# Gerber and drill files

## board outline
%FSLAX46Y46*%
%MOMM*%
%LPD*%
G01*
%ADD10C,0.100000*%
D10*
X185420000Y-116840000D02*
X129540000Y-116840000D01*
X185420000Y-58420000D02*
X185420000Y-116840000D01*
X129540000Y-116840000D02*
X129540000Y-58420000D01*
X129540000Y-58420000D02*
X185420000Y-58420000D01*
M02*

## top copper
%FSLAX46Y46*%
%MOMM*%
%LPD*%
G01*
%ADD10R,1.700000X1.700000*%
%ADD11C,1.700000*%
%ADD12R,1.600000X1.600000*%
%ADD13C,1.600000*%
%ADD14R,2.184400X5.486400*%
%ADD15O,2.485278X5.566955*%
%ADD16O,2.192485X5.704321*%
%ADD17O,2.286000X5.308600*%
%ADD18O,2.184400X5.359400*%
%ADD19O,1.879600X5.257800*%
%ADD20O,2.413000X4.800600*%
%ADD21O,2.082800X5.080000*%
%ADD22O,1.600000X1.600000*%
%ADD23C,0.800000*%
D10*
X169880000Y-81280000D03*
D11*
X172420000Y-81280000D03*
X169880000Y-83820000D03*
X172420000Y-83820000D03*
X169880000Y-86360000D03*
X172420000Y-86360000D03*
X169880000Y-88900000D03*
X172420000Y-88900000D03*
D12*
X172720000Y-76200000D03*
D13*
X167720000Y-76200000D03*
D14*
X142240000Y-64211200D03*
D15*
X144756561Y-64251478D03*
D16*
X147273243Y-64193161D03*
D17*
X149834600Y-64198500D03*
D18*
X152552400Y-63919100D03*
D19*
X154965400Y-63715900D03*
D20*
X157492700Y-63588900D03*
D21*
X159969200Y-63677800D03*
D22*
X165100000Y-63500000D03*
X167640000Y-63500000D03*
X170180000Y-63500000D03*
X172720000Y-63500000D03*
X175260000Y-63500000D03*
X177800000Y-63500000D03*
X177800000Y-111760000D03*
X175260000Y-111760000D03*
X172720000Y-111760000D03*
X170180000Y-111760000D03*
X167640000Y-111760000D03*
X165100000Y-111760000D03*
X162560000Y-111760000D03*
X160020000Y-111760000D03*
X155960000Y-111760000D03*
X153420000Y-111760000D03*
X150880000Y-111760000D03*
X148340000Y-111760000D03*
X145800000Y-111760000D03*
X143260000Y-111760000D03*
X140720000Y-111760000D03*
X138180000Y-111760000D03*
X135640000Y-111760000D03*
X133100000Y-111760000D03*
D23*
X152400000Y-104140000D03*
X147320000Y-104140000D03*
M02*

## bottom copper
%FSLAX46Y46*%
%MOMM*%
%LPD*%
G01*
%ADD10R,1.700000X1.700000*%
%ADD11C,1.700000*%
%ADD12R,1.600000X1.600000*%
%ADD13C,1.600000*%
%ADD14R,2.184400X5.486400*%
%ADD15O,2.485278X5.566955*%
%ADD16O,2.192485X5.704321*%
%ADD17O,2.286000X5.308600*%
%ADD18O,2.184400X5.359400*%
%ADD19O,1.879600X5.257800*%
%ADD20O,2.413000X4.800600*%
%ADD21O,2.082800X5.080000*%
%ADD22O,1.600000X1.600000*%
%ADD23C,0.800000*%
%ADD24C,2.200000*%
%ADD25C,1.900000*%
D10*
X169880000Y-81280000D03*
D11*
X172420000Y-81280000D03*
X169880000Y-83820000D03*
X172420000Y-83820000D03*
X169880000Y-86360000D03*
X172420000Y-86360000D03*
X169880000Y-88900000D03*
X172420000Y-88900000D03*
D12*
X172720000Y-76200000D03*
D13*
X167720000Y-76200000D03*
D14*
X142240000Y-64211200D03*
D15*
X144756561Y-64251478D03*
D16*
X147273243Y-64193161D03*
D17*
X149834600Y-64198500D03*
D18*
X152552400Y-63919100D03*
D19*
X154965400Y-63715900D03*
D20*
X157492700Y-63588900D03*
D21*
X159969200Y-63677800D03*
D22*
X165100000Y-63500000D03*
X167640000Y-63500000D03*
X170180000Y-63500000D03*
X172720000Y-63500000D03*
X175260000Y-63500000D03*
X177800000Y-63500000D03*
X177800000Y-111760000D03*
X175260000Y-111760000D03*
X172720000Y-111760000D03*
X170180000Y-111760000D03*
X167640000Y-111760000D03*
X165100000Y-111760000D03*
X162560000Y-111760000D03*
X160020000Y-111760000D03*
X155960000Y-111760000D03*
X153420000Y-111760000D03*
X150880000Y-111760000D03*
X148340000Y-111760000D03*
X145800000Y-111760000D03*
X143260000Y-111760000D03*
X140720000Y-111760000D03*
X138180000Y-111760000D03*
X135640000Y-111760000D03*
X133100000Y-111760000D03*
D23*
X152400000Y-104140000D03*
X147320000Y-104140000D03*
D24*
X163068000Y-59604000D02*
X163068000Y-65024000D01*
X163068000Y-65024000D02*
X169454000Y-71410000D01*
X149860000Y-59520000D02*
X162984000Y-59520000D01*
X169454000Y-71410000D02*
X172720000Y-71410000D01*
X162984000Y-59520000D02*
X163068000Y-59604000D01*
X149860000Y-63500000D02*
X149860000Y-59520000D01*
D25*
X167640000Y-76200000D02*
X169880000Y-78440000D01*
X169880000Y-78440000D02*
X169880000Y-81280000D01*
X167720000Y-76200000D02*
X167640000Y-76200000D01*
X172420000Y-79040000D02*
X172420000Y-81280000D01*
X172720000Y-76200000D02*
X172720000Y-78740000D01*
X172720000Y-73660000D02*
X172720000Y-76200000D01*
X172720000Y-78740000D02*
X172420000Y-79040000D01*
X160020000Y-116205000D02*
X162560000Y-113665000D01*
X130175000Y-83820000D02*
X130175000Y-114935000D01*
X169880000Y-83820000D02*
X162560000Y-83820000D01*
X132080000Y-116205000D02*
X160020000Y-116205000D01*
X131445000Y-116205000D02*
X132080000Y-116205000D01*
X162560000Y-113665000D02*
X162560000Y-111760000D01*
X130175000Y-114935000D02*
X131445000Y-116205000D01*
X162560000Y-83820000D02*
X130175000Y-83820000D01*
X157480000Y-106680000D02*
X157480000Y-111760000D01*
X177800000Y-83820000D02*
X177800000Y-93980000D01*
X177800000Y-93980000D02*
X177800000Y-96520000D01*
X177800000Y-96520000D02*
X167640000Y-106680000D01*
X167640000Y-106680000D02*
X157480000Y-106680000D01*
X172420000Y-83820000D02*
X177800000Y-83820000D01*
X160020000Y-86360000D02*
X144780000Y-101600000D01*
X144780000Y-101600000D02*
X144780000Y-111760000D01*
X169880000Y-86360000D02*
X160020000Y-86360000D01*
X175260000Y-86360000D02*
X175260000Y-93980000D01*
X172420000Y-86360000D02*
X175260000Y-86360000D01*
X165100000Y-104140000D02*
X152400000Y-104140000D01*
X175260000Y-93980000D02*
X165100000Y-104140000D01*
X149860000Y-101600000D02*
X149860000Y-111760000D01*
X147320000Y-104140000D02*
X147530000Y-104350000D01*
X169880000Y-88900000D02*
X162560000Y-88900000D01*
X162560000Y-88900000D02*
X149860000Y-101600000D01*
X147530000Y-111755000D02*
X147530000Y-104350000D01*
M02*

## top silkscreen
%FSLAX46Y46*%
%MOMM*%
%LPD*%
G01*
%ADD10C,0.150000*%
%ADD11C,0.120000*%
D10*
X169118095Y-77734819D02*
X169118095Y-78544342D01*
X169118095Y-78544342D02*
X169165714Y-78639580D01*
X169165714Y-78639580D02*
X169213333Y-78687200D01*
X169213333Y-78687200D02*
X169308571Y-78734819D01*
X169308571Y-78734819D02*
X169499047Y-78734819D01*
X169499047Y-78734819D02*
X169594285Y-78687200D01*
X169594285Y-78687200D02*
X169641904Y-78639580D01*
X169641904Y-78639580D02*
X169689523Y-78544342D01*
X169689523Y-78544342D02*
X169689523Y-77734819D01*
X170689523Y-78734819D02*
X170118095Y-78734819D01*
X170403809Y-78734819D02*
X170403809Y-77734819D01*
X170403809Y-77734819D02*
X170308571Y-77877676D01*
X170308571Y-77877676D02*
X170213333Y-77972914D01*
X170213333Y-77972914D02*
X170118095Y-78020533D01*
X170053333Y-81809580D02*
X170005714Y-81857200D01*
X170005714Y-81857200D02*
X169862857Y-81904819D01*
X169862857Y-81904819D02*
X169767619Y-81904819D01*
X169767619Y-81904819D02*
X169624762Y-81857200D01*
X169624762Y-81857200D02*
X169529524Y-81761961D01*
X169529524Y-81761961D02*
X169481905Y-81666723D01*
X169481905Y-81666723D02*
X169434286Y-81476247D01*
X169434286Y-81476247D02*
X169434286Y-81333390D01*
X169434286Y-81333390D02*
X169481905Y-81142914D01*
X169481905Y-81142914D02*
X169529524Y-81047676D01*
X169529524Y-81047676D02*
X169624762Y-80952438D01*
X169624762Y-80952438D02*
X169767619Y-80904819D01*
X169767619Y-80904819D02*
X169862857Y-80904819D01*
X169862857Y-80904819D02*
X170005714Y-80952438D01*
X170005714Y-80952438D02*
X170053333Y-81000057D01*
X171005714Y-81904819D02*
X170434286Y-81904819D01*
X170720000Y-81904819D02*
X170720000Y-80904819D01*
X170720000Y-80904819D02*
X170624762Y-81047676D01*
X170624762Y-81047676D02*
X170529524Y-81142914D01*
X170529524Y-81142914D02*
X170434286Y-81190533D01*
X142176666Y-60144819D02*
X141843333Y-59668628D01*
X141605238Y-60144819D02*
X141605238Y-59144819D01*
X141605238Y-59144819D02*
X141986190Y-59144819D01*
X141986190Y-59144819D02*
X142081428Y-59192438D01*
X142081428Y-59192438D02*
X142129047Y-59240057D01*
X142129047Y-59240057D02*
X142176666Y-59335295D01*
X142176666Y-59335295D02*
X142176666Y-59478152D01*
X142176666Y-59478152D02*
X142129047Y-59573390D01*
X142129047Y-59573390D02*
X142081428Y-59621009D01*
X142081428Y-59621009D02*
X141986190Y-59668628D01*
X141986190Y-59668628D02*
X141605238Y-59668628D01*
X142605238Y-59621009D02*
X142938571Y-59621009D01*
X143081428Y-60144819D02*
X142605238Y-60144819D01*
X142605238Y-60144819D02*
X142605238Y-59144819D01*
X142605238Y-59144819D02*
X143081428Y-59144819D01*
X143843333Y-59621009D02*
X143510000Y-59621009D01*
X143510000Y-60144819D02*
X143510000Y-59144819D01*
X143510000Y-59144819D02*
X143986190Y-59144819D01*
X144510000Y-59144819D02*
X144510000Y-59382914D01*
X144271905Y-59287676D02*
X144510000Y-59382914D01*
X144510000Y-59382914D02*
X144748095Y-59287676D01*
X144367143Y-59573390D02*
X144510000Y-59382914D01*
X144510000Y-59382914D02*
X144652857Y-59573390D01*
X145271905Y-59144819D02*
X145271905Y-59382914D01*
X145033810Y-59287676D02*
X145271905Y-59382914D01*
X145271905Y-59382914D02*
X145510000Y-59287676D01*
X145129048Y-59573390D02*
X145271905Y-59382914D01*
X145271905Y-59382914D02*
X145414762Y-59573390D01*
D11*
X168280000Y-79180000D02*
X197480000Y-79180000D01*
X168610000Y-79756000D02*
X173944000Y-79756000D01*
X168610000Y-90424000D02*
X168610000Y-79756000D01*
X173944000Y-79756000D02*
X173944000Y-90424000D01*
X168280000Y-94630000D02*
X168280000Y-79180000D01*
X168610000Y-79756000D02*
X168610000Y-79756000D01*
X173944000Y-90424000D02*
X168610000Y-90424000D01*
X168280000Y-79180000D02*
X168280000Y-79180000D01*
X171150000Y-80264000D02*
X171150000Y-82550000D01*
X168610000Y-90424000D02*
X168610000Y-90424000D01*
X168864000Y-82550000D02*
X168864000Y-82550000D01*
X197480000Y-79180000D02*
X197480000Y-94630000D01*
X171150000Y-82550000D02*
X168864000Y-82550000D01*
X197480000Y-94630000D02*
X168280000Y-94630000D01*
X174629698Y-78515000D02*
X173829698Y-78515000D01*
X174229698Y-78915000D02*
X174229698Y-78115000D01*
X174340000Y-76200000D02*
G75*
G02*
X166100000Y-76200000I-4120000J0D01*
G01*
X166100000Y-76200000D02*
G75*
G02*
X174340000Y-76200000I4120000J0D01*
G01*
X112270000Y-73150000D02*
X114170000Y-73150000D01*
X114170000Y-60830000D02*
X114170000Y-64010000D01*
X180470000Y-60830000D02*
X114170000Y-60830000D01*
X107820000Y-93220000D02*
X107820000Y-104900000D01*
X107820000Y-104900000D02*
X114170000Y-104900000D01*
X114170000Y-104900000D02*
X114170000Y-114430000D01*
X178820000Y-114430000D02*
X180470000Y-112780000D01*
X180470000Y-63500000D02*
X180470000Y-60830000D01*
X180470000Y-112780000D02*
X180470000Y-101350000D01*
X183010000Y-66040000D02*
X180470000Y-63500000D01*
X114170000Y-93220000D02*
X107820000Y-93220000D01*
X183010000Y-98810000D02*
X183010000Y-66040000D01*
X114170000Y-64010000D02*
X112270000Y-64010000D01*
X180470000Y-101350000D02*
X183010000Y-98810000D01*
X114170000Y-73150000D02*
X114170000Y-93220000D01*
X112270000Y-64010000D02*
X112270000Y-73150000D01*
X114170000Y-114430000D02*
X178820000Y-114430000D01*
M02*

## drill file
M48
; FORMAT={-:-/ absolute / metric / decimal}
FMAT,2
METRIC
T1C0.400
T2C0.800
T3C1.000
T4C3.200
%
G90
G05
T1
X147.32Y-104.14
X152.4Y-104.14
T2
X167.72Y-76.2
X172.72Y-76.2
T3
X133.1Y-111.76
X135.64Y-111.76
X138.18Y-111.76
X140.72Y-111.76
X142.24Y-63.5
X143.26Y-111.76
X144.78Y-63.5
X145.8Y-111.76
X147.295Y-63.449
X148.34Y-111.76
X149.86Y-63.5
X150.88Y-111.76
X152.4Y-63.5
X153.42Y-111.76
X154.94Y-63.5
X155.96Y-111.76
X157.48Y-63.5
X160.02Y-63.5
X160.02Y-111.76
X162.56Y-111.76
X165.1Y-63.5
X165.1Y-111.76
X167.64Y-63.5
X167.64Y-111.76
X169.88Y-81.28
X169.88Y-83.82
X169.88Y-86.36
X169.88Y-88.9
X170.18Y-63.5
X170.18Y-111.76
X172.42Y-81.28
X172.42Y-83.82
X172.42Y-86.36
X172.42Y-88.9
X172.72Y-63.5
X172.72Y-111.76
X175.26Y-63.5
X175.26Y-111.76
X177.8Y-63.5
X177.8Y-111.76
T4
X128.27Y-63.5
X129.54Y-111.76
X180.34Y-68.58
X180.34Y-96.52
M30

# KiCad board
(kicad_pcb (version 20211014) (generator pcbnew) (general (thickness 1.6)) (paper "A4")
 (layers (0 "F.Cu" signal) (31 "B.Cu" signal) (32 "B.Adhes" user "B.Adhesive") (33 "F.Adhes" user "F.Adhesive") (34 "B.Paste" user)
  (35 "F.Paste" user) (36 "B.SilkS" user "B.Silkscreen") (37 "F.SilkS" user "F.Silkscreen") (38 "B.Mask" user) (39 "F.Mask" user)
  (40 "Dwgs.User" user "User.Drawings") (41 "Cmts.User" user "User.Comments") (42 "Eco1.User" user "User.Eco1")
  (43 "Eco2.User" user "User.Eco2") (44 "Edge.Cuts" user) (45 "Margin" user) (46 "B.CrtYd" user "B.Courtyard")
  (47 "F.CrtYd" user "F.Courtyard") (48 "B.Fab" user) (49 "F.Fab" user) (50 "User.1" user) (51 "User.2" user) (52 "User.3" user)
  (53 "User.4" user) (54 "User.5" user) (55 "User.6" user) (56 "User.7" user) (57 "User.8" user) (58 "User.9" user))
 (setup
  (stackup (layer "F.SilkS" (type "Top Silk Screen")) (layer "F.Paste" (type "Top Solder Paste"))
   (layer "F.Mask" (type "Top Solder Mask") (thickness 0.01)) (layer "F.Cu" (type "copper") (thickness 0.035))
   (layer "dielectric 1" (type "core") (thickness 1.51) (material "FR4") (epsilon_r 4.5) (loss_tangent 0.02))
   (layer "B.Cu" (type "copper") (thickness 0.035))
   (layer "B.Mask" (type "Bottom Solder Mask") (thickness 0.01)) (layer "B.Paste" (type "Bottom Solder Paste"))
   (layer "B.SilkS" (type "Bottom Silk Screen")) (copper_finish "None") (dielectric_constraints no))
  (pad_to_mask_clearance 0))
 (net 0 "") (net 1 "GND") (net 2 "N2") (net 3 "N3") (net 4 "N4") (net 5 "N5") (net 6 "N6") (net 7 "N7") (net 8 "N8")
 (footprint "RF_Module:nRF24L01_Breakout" (layer "F.Cu") (at 169.88 81.28)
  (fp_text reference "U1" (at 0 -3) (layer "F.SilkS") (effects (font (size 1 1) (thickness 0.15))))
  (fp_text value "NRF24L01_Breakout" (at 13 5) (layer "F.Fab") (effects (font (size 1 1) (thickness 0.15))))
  (fp_line (start -1.6 -2.1) (end 27.6 -2.1) (layer "F.SilkS") (width 0.12))
  (fp_line (start -1.27 -1.524) (end 4.064 -1.524) (layer "F.SilkS") (width 0.12))
  (fp_line (start -1.27 9.144) (end -1.27 -1.524) (layer "F.SilkS") (width 0.12))
  (fp_line (start 4.064 -1.524) (end 4.064 9.144) (layer "F.SilkS") (width 0.12))
  (fp_line (start -1.6 13.35) (end -1.6 -2.1) (layer "F.SilkS") (width 0.12))
  (fp_line (start -1.27 -1.524) (end -1.27 -1.524) (layer "F.SilkS") (width 0.12))
  (fp_line (start 4.064 9.144) (end -1.27 9.144) (layer "F.SilkS") (width 0.12))
  (fp_line (start -1.6 -2.1) (end -1.6 -2.1) (layer "F.SilkS") (width 0.12))
  (fp_line (start 1.27 -1.016) (end 1.27 1.27) (layer "F.SilkS") (width 0.12))
  (fp_line (start -1.27 9.144) (end -1.27 9.144) (layer "F.SilkS") (width 0.12))
  (fp_line (start -1.016 1.27) (end -1.016 1.27) (layer "F.SilkS") (width 0.12))
  (fp_line (start 27.6 -2.1) (end 27.6 13.35) (layer "F.SilkS") (width 0.12))
  (fp_line (start 1.27 1.27) (end -1.016 1.27) (layer "F.SilkS") (width 0.12))
  (fp_line (start 27.6 13.35) (end -1.6 13.35) (layer "F.SilkS") (width 0.12))
  (pad "1" thru_hole rect (at 0 0) (size 1.7 1.7) (drill 1) (layers *.Cu *.Mask) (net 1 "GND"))
  (pad "2" thru_hole circle (at 2.54 0) (size 1.7 1.7) (drill 1) (layers *.Cu *.Mask) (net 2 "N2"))
  (pad "3" thru_hole circle (at 0 2.54) (size 1.7 1.7) (drill 1) (layers *.Cu *.Mask) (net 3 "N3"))
  (pad "4" thru_hole circle (at 2.54 2.54) (size 1.7 1.7) (drill 1) (layers *.Cu *.Mask) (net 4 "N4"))
  (pad "5" thru_hole circle (at 0 5.08) (size 1.7 1.7) (drill 1) (layers *.Cu *.Mask) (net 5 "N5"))
  (pad "6" thru_hole circle (at 2.54 5.08) (size 1.7 1.7) (drill 1) (layers *.Cu *.Mask) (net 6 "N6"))
  (pad "7" thru_hole circle (at 0 7.62) (size 1.7 1.7) (drill 1) (layers *.Cu *.Mask) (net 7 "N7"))
  (pad "8" thru_hole circle (at 2.54 7.62) (size 1.7 1.7) (drill 1) (layers *.Cu *.Mask) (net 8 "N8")))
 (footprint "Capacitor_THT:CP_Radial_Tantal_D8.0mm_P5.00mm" (layer "F.Cu") (at 172.72 76.2 180)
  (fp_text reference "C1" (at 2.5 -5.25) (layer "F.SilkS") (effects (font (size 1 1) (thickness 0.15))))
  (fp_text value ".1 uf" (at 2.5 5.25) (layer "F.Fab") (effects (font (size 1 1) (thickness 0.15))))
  (fp_line (start -1.909698 -2.315) (end -1.109698 -2.315) (layer "F.SilkS") (width 0.12))
  (fp_line (start -1.509698 -2.715) (end -1.509698 -1.915) (layer "F.SilkS") (width 0.12))
  (fp_circle (center 2.5 0) (end 6.62 0) (layer "F.SilkS") (width 0.12) (fill none))
  (pad "1" thru_hole rect (at 0 0 180) (size 1.6 1.6) (drill 0.8) (layers *.Cu *.Mask) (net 2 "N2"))
  (pad "2" thru_hole circle (at 5 0 180) (size 1.6 1.6) (drill 0.8) (layers *.Cu *.Mask) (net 1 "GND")))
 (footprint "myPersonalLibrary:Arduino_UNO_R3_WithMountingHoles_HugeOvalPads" (layer "F.Cu") (at 142.24 63.5)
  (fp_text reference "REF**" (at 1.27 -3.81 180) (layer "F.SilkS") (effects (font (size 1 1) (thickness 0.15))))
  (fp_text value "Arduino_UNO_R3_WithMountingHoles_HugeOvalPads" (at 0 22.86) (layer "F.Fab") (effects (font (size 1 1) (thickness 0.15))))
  (fp_line (start -29.97 9.65) (end -28.07 9.65) (layer "F.SilkS") (width 0.12))
  (fp_line (start -28.07 -2.67) (end -28.07 0.51) (layer "F.SilkS") (width 0.12))
  (fp_line (start 38.23 -2.67) (end -28.07 -2.67) (layer "F.SilkS") (width 0.12))
  (fp_line (start -34.42 29.72) (end -34.42 41.4) (layer "F.SilkS") (width 0.12))
  (fp_line (start -34.42 41.4) (end -28.07 41.4) (layer "F.SilkS") (width 0.12))
  (fp_line (start -28.07 41.4) (end -28.07 50.93) (layer "F.SilkS") (width 0.12))
  (fp_line (start 36.58 50.93) (end 38.23 49.28) (layer "F.SilkS") (width 0.12))
  (fp_line (start 38.23 0) (end 38.23 -2.67) (layer "F.SilkS") (width 0.12))
  (fp_line (start 38.23 49.28) (end 38.23 37.85) (layer "F.SilkS") (width 0.12))
  (fp_line (start 40.77 2.54) (end 38.23 0) (layer "F.SilkS") (width 0.12))
  (fp_line (start -28.07 29.72) (end -34.42 29.72) (layer "F.SilkS") (width 0.12))
  (fp_line (start 40.77 35.31) (end 40.77 2.54) (layer "F.SilkS") (width 0.12))
  (fp_line (start -28.07 0.51) (end -29.97 0.51) (layer "F.SilkS") (width 0.12))
  (fp_line (start 38.23 37.85) (end 40.77 35.31) (layer "F.SilkS") (width 0.12))
  (fp_line (start -28.07 9.65) (end -28.07 29.72) (layer "F.SilkS") (width 0.12))
  (fp_line (start -29.97 0.51) (end -29.97 9.65) (layer "F.SilkS") (width 0.12))
  (fp_line (start -28.07 50.93) (end 36.58 50.93) (layer "F.SilkS") (width 0.12))
  (pad "" np_thru_hole circle (at -12.7 48.26 90) (size 3.2 3.2) (drill 3.2) (layers *.Cu *.Mask))
  (pad "" np_thru_hole circle (at 38.1 5.08 90) (size 3.2 3.2) (drill 3.2) (layers *.Cu *.Mask))
  (pad "" np_thru_hole circle (at -13.97 0 90) (size 3.2 3.2) (drill 3.2) (layers *.Cu *.Mask))
  (pad "" np_thru_hole circle (at 38.1 33.02 90) (size 3.2 3.2) (drill 3.2) (layers *.Cu *.Mask))
  (pad "1" thru_hole rect (at 0 0 90) (size 5.4864 2.1844) (drill 1 (offset -0.7112 0)) (layers *.Cu *.Mask))
  (pad "2" thru_hole oval (at 2.54 0 90) (size 5.566955 2.485278) (drill 1 (offset -0.751478 -0.023439)) (layers *.Cu *.Mask))
  (pad "3" thru_hole oval (at 5.0546 -0.0508 90) (size 5.704321 2.192485) (drill 1 (offset -0.743961 -0.021357)) (layers *.Cu *.Mask))
  (pad "4" thru_hole oval (at 7.62 0 90) (size 5.3086 2.286) (drill 1 (offset -0.6985 -0.0254)) (layers *.Cu *.Mask))
  (pad "5" thru_hole oval (at 10.16 0 90) (size 5.3594 2.1844) (drill 1 (offset -0.4191 0.1524)) (layers *.Cu *.Mask))
  (pad "6" thru_hole oval (at 12.7 0 90) (size 5.2578 1.8796) (drill 1 (offset -0.2159 0.0254)) (layers *.Cu *.Mask))
  (pad "7" thru_hole oval (at 15.24 0 90) (size 4.8006 2.413) (drill 1 (offset -0.0889 0.0127)) (layers *.Cu *.Mask))
  (pad "8" thru_hole oval (at 17.78 0 90) (size 5.08 2.0828) (drill 1 (offset -0.1778 -0.0508)) (layers *.Cu *.Mask))
  (pad "9" thru_hole oval (at 22.86 0 90) (size 1.6 1.6) (drill 1) (layers *.Cu *.Mask))
  (pad "10" thru_hole oval (at 25.4 0 90) (size 1.6 1.6) (drill 1) (layers *.Cu *.Mask))
  (pad "11" thru_hole oval (at 27.94 0 90) (size 1.6 1.6) (drill 1) (layers *.Cu *.Mask))
  (pad "12" thru_hole oval (at 30.48 0 90) (size 1.6 1.6) (drill 1) (layers *.Cu *.Mask))
  (pad "13" thru_hole oval (at 33.02 0 90) (size 1.6 1.6) (drill 1) (layers *.Cu *.Mask))
  (pad "14" thru_hole oval (at 35.56 0 90) (size 1.6 1.6) (drill 1) (layers *.Cu *.Mask))
  (pad "15" thru_hole oval (at 35.56 48.26 90) (size 1.6 1.6) (drill 1) (layers *.Cu *.Mask))
  (pad "16" thru_hole oval (at 33.02 48.26 90) (size 1.6 1.6) (drill 1) (layers *.Cu *.Mask))
  (pad "17" thru_hole oval (at 30.48 48.26 90) (size 1.6 1.6) (drill 1) (layers *.Cu *.Mask))
  (pad "18" thru_hole oval (at 27.94 48.26 90) (size 1.6 1.6) (drill 1) (layers *.Cu *.Mask))
  (pad "19" thru_hole oval (at 25.4 48.26 90) (size 1.6 1.6) (drill 1) (layers *.Cu *.Mask))
  (pad "20" thru_hole oval (at 22.86 48.26 90) (size 1.6 1.6) (drill 1) (layers *.Cu *.Mask))
  (pad "21" thru_hole oval (at 20.32 48.26 90) (size 1.6 1.6) (drill 1) (layers *.Cu *.Mask))
  (pad "22" thru_hole oval (at 17.78 48.26 90) (size 1.6 1.6) (drill 1) (layers *.Cu *.Mask))
  (pad "23" thru_hole oval (at 13.72 48.26 90) (size 1.6 1.6) (drill 1) (layers *.Cu *.Mask))
  (pad "24" thru_hole oval (at 11.18 48.26 90) (size 1.6 1.6) (drill 1) (layers *.Cu *.Mask))
  (pad "25" thru_hole oval (at 8.64 48.26 90) (size 1.6 1.6) (drill 1) (layers *.Cu *.Mask))
  (pad "26" thru_hole oval (at 6.1 48.26 90) (size 1.6 1.6) (drill 1) (layers *.Cu *.Mask))
  (pad "27" thru_hole oval (at 3.56 48.26 90) (size 1.6 1.6) (drill 1) (layers *.Cu *.Mask))
  (pad "28" thru_hole oval (at 1.02 48.26 90) (size 1.6 1.6) (drill 1) (layers *.Cu *.Mask))
  (pad "29" thru_hole oval (at -1.52 48.26 90) (size 1.6 1.6) (drill 1) (layers *.Cu *.Mask))
  (pad "30" thru_hole oval (at -4.06 48.26 90) (size 1.6 1.6) (drill 1) (layers *.Cu *.Mask))
  (pad "31" thru_hole oval (at -6.6 48.26 90) (size 1.6 1.6) (drill 1) (layers *.Cu *.Mask))
  (pad "32" thru_hole oval (at -9.14 48.26 90) (size 1.6 1.6) (drill 1) (layers *.Cu *.Mask)))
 (gr_line (start 185.42 116.84) (end 129.54 116.84) (layer "Edge.Cuts") (width 0.1))
 (gr_line (start 185.42 58.42) (end 185.42 116.84) (layer "Edge.Cuts") (width 0.1))
 (gr_line (start 129.54 116.84) (end 129.54 58.42) (layer "Edge.Cuts") (width 0.1))
 (gr_line (start 129.54 58.42) (end 185.42 58.42) (layer "Edge.Cuts") (width 0.1))
 (segment (start 163.068 59.604) (end 163.068 65.024) (width 2.2) (layer "B.Cu") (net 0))
 (segment (start 163.068 65.024) (end 169.454 71.41) (width 2.2) (layer "B.Cu") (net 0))
 (segment (start 149.86 59.52) (end 162.984 59.52) (width 2.2) (layer "B.Cu") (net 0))
 (segment (start 169.454 71.41) (end 172.72 71.41) (width 2.2) (layer "B.Cu") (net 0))
 (segment (start 162.984 59.52) (end 163.068 59.604) (width 2.2) (layer "B.Cu") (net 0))
 (segment (start 149.86 63.5) (end 149.86 59.52) (width 2.2) (layer "B.Cu") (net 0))
 (segment (start 167.64 76.2) (end 169.88 78.44) (width 1.9) (layer "B.Cu") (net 1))
 (segment (start 169.88 78.44) (end 169.88 81.28) (width 1.9) (layer "B.Cu") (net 1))
 (segment (start 167.72 76.2) (end 167.64 76.2) (width 1.9) (layer "B.Cu") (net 1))
 (segment (start 172.42 79.04) (end 172.42 81.28) (width 1.9) (layer "B.Cu") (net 2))
 (segment (start 172.72 76.2) (end 172.72 78.74) (width 1.9) (layer "B.Cu") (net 2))
 (segment (start 172.72 73.66) (end 172.72 76.2) (width 1.9) (layer "B.Cu") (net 2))
 (segment (start 172.72 78.74) (end 172.42 79.04) (width 1.9) (layer "B.Cu") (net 2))
 (segment (start 160.02 116.205) (end 162.56 113.665) (width 1.9) (layer "B.Cu") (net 3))
 (segment (start 130.175 83.82) (end 130.175 114.935) (width 1.9) (layer "B.Cu") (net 3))
 (segment (start 169.88 83.82) (end 162.56 83.82) (width 1.9) (layer "B.Cu") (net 3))
 (segment (start 132.08 116.205) (end 160.02 116.205) (width 1.9) (layer "B.Cu") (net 3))
 (segment (start 131.445 116.205) (end 132.08 116.205) (width 1.9) (layer "B.Cu") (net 3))
 (segment (start 162.56 113.665) (end 162.56 111.76) (width 1.9) (layer "B.Cu") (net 3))
 (segment (start 130.175 114.935) (end 131.445 116.205) (width 1.9) (layer "B.Cu") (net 3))
 (segment (start 162.56 83.82) (end 130.175 83.82) (width 1.9) (layer "B.Cu") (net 3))
 (segment (start 157.48 106.68) (end 157.48 111.76) (width 1.9) (layer "B.Cu") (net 4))
 (segment (start 177.8 83.82) (end 177.8 93.98) (width 1.9) (layer "B.Cu") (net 4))
 (segment (start 177.8 93.98) (end 177.8 96.52) (width 1.9) (layer "B.Cu") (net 4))
 (segment (start 177.8 96.52) (end 167.64 106.68) (width 1.9) (layer "B.Cu") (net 4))
 (segment (start 167.64 106.68) (end 157.48 106.68) (width 1.9) (layer "B.Cu") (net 4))
 (segment (start 172.42 83.82) (end 177.8 83.82) (width 1.9) (layer "B.Cu") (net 4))
 (segment (start 160.02 86.36) (end 144.78 101.6) (width 1.9) (layer "B.Cu") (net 5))
 (segment (start 144.78 101.6) (end 144.78 111.76) (width 1.9) (layer "B.Cu") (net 5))
 (segment (start 169.88 86.36) (end 160.02 86.36) (width 1.9) (layer "B.Cu") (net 5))
 (via (at 152.4 104.14) (size 0.8) (drill 0.4) (layers "F.Cu" "B.Cu") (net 6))
 (segment (start 175.26 86.36) (end 175.26 93.98) (width 1.9) (layer "B.Cu") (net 6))
 (segment (start 172.42 86.36) (end 175.26 86.36) (width 1.9) (layer "B.Cu") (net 6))
 (segment (start 165.1 104.14) (end 152.4 104.14) (width 1.9) (layer "B.Cu") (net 6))
 (segment (start 175.26 93.98) (end 165.1 104.14) (width 1.9) (layer "B.Cu") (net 6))
 (via (at 147.32 104.14) (size 0.8) (drill 0.4) (layers "F.Cu" "B.Cu") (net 7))
 (segment (start 149.86 101.6) (end 149.86 111.76) (width 1.9) (layer "B.Cu") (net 7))
 (segment (start 147.32 104.14) (end 147.53 104.35) (width 1.9) (layer "B.Cu") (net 7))
 (segment (start 169.88 88.9) (end 162.56 88.9) (width 1.9) (layer "B.Cu") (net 7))
 (segment (start 162.56 88.9) (end 149.86 101.6) (width 1.9) (layer "B.Cu") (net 7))
 (segment (start 147.53 111.755) (end 147.53 104.35) (width 1.9) (layer "B.Cu") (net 7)))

